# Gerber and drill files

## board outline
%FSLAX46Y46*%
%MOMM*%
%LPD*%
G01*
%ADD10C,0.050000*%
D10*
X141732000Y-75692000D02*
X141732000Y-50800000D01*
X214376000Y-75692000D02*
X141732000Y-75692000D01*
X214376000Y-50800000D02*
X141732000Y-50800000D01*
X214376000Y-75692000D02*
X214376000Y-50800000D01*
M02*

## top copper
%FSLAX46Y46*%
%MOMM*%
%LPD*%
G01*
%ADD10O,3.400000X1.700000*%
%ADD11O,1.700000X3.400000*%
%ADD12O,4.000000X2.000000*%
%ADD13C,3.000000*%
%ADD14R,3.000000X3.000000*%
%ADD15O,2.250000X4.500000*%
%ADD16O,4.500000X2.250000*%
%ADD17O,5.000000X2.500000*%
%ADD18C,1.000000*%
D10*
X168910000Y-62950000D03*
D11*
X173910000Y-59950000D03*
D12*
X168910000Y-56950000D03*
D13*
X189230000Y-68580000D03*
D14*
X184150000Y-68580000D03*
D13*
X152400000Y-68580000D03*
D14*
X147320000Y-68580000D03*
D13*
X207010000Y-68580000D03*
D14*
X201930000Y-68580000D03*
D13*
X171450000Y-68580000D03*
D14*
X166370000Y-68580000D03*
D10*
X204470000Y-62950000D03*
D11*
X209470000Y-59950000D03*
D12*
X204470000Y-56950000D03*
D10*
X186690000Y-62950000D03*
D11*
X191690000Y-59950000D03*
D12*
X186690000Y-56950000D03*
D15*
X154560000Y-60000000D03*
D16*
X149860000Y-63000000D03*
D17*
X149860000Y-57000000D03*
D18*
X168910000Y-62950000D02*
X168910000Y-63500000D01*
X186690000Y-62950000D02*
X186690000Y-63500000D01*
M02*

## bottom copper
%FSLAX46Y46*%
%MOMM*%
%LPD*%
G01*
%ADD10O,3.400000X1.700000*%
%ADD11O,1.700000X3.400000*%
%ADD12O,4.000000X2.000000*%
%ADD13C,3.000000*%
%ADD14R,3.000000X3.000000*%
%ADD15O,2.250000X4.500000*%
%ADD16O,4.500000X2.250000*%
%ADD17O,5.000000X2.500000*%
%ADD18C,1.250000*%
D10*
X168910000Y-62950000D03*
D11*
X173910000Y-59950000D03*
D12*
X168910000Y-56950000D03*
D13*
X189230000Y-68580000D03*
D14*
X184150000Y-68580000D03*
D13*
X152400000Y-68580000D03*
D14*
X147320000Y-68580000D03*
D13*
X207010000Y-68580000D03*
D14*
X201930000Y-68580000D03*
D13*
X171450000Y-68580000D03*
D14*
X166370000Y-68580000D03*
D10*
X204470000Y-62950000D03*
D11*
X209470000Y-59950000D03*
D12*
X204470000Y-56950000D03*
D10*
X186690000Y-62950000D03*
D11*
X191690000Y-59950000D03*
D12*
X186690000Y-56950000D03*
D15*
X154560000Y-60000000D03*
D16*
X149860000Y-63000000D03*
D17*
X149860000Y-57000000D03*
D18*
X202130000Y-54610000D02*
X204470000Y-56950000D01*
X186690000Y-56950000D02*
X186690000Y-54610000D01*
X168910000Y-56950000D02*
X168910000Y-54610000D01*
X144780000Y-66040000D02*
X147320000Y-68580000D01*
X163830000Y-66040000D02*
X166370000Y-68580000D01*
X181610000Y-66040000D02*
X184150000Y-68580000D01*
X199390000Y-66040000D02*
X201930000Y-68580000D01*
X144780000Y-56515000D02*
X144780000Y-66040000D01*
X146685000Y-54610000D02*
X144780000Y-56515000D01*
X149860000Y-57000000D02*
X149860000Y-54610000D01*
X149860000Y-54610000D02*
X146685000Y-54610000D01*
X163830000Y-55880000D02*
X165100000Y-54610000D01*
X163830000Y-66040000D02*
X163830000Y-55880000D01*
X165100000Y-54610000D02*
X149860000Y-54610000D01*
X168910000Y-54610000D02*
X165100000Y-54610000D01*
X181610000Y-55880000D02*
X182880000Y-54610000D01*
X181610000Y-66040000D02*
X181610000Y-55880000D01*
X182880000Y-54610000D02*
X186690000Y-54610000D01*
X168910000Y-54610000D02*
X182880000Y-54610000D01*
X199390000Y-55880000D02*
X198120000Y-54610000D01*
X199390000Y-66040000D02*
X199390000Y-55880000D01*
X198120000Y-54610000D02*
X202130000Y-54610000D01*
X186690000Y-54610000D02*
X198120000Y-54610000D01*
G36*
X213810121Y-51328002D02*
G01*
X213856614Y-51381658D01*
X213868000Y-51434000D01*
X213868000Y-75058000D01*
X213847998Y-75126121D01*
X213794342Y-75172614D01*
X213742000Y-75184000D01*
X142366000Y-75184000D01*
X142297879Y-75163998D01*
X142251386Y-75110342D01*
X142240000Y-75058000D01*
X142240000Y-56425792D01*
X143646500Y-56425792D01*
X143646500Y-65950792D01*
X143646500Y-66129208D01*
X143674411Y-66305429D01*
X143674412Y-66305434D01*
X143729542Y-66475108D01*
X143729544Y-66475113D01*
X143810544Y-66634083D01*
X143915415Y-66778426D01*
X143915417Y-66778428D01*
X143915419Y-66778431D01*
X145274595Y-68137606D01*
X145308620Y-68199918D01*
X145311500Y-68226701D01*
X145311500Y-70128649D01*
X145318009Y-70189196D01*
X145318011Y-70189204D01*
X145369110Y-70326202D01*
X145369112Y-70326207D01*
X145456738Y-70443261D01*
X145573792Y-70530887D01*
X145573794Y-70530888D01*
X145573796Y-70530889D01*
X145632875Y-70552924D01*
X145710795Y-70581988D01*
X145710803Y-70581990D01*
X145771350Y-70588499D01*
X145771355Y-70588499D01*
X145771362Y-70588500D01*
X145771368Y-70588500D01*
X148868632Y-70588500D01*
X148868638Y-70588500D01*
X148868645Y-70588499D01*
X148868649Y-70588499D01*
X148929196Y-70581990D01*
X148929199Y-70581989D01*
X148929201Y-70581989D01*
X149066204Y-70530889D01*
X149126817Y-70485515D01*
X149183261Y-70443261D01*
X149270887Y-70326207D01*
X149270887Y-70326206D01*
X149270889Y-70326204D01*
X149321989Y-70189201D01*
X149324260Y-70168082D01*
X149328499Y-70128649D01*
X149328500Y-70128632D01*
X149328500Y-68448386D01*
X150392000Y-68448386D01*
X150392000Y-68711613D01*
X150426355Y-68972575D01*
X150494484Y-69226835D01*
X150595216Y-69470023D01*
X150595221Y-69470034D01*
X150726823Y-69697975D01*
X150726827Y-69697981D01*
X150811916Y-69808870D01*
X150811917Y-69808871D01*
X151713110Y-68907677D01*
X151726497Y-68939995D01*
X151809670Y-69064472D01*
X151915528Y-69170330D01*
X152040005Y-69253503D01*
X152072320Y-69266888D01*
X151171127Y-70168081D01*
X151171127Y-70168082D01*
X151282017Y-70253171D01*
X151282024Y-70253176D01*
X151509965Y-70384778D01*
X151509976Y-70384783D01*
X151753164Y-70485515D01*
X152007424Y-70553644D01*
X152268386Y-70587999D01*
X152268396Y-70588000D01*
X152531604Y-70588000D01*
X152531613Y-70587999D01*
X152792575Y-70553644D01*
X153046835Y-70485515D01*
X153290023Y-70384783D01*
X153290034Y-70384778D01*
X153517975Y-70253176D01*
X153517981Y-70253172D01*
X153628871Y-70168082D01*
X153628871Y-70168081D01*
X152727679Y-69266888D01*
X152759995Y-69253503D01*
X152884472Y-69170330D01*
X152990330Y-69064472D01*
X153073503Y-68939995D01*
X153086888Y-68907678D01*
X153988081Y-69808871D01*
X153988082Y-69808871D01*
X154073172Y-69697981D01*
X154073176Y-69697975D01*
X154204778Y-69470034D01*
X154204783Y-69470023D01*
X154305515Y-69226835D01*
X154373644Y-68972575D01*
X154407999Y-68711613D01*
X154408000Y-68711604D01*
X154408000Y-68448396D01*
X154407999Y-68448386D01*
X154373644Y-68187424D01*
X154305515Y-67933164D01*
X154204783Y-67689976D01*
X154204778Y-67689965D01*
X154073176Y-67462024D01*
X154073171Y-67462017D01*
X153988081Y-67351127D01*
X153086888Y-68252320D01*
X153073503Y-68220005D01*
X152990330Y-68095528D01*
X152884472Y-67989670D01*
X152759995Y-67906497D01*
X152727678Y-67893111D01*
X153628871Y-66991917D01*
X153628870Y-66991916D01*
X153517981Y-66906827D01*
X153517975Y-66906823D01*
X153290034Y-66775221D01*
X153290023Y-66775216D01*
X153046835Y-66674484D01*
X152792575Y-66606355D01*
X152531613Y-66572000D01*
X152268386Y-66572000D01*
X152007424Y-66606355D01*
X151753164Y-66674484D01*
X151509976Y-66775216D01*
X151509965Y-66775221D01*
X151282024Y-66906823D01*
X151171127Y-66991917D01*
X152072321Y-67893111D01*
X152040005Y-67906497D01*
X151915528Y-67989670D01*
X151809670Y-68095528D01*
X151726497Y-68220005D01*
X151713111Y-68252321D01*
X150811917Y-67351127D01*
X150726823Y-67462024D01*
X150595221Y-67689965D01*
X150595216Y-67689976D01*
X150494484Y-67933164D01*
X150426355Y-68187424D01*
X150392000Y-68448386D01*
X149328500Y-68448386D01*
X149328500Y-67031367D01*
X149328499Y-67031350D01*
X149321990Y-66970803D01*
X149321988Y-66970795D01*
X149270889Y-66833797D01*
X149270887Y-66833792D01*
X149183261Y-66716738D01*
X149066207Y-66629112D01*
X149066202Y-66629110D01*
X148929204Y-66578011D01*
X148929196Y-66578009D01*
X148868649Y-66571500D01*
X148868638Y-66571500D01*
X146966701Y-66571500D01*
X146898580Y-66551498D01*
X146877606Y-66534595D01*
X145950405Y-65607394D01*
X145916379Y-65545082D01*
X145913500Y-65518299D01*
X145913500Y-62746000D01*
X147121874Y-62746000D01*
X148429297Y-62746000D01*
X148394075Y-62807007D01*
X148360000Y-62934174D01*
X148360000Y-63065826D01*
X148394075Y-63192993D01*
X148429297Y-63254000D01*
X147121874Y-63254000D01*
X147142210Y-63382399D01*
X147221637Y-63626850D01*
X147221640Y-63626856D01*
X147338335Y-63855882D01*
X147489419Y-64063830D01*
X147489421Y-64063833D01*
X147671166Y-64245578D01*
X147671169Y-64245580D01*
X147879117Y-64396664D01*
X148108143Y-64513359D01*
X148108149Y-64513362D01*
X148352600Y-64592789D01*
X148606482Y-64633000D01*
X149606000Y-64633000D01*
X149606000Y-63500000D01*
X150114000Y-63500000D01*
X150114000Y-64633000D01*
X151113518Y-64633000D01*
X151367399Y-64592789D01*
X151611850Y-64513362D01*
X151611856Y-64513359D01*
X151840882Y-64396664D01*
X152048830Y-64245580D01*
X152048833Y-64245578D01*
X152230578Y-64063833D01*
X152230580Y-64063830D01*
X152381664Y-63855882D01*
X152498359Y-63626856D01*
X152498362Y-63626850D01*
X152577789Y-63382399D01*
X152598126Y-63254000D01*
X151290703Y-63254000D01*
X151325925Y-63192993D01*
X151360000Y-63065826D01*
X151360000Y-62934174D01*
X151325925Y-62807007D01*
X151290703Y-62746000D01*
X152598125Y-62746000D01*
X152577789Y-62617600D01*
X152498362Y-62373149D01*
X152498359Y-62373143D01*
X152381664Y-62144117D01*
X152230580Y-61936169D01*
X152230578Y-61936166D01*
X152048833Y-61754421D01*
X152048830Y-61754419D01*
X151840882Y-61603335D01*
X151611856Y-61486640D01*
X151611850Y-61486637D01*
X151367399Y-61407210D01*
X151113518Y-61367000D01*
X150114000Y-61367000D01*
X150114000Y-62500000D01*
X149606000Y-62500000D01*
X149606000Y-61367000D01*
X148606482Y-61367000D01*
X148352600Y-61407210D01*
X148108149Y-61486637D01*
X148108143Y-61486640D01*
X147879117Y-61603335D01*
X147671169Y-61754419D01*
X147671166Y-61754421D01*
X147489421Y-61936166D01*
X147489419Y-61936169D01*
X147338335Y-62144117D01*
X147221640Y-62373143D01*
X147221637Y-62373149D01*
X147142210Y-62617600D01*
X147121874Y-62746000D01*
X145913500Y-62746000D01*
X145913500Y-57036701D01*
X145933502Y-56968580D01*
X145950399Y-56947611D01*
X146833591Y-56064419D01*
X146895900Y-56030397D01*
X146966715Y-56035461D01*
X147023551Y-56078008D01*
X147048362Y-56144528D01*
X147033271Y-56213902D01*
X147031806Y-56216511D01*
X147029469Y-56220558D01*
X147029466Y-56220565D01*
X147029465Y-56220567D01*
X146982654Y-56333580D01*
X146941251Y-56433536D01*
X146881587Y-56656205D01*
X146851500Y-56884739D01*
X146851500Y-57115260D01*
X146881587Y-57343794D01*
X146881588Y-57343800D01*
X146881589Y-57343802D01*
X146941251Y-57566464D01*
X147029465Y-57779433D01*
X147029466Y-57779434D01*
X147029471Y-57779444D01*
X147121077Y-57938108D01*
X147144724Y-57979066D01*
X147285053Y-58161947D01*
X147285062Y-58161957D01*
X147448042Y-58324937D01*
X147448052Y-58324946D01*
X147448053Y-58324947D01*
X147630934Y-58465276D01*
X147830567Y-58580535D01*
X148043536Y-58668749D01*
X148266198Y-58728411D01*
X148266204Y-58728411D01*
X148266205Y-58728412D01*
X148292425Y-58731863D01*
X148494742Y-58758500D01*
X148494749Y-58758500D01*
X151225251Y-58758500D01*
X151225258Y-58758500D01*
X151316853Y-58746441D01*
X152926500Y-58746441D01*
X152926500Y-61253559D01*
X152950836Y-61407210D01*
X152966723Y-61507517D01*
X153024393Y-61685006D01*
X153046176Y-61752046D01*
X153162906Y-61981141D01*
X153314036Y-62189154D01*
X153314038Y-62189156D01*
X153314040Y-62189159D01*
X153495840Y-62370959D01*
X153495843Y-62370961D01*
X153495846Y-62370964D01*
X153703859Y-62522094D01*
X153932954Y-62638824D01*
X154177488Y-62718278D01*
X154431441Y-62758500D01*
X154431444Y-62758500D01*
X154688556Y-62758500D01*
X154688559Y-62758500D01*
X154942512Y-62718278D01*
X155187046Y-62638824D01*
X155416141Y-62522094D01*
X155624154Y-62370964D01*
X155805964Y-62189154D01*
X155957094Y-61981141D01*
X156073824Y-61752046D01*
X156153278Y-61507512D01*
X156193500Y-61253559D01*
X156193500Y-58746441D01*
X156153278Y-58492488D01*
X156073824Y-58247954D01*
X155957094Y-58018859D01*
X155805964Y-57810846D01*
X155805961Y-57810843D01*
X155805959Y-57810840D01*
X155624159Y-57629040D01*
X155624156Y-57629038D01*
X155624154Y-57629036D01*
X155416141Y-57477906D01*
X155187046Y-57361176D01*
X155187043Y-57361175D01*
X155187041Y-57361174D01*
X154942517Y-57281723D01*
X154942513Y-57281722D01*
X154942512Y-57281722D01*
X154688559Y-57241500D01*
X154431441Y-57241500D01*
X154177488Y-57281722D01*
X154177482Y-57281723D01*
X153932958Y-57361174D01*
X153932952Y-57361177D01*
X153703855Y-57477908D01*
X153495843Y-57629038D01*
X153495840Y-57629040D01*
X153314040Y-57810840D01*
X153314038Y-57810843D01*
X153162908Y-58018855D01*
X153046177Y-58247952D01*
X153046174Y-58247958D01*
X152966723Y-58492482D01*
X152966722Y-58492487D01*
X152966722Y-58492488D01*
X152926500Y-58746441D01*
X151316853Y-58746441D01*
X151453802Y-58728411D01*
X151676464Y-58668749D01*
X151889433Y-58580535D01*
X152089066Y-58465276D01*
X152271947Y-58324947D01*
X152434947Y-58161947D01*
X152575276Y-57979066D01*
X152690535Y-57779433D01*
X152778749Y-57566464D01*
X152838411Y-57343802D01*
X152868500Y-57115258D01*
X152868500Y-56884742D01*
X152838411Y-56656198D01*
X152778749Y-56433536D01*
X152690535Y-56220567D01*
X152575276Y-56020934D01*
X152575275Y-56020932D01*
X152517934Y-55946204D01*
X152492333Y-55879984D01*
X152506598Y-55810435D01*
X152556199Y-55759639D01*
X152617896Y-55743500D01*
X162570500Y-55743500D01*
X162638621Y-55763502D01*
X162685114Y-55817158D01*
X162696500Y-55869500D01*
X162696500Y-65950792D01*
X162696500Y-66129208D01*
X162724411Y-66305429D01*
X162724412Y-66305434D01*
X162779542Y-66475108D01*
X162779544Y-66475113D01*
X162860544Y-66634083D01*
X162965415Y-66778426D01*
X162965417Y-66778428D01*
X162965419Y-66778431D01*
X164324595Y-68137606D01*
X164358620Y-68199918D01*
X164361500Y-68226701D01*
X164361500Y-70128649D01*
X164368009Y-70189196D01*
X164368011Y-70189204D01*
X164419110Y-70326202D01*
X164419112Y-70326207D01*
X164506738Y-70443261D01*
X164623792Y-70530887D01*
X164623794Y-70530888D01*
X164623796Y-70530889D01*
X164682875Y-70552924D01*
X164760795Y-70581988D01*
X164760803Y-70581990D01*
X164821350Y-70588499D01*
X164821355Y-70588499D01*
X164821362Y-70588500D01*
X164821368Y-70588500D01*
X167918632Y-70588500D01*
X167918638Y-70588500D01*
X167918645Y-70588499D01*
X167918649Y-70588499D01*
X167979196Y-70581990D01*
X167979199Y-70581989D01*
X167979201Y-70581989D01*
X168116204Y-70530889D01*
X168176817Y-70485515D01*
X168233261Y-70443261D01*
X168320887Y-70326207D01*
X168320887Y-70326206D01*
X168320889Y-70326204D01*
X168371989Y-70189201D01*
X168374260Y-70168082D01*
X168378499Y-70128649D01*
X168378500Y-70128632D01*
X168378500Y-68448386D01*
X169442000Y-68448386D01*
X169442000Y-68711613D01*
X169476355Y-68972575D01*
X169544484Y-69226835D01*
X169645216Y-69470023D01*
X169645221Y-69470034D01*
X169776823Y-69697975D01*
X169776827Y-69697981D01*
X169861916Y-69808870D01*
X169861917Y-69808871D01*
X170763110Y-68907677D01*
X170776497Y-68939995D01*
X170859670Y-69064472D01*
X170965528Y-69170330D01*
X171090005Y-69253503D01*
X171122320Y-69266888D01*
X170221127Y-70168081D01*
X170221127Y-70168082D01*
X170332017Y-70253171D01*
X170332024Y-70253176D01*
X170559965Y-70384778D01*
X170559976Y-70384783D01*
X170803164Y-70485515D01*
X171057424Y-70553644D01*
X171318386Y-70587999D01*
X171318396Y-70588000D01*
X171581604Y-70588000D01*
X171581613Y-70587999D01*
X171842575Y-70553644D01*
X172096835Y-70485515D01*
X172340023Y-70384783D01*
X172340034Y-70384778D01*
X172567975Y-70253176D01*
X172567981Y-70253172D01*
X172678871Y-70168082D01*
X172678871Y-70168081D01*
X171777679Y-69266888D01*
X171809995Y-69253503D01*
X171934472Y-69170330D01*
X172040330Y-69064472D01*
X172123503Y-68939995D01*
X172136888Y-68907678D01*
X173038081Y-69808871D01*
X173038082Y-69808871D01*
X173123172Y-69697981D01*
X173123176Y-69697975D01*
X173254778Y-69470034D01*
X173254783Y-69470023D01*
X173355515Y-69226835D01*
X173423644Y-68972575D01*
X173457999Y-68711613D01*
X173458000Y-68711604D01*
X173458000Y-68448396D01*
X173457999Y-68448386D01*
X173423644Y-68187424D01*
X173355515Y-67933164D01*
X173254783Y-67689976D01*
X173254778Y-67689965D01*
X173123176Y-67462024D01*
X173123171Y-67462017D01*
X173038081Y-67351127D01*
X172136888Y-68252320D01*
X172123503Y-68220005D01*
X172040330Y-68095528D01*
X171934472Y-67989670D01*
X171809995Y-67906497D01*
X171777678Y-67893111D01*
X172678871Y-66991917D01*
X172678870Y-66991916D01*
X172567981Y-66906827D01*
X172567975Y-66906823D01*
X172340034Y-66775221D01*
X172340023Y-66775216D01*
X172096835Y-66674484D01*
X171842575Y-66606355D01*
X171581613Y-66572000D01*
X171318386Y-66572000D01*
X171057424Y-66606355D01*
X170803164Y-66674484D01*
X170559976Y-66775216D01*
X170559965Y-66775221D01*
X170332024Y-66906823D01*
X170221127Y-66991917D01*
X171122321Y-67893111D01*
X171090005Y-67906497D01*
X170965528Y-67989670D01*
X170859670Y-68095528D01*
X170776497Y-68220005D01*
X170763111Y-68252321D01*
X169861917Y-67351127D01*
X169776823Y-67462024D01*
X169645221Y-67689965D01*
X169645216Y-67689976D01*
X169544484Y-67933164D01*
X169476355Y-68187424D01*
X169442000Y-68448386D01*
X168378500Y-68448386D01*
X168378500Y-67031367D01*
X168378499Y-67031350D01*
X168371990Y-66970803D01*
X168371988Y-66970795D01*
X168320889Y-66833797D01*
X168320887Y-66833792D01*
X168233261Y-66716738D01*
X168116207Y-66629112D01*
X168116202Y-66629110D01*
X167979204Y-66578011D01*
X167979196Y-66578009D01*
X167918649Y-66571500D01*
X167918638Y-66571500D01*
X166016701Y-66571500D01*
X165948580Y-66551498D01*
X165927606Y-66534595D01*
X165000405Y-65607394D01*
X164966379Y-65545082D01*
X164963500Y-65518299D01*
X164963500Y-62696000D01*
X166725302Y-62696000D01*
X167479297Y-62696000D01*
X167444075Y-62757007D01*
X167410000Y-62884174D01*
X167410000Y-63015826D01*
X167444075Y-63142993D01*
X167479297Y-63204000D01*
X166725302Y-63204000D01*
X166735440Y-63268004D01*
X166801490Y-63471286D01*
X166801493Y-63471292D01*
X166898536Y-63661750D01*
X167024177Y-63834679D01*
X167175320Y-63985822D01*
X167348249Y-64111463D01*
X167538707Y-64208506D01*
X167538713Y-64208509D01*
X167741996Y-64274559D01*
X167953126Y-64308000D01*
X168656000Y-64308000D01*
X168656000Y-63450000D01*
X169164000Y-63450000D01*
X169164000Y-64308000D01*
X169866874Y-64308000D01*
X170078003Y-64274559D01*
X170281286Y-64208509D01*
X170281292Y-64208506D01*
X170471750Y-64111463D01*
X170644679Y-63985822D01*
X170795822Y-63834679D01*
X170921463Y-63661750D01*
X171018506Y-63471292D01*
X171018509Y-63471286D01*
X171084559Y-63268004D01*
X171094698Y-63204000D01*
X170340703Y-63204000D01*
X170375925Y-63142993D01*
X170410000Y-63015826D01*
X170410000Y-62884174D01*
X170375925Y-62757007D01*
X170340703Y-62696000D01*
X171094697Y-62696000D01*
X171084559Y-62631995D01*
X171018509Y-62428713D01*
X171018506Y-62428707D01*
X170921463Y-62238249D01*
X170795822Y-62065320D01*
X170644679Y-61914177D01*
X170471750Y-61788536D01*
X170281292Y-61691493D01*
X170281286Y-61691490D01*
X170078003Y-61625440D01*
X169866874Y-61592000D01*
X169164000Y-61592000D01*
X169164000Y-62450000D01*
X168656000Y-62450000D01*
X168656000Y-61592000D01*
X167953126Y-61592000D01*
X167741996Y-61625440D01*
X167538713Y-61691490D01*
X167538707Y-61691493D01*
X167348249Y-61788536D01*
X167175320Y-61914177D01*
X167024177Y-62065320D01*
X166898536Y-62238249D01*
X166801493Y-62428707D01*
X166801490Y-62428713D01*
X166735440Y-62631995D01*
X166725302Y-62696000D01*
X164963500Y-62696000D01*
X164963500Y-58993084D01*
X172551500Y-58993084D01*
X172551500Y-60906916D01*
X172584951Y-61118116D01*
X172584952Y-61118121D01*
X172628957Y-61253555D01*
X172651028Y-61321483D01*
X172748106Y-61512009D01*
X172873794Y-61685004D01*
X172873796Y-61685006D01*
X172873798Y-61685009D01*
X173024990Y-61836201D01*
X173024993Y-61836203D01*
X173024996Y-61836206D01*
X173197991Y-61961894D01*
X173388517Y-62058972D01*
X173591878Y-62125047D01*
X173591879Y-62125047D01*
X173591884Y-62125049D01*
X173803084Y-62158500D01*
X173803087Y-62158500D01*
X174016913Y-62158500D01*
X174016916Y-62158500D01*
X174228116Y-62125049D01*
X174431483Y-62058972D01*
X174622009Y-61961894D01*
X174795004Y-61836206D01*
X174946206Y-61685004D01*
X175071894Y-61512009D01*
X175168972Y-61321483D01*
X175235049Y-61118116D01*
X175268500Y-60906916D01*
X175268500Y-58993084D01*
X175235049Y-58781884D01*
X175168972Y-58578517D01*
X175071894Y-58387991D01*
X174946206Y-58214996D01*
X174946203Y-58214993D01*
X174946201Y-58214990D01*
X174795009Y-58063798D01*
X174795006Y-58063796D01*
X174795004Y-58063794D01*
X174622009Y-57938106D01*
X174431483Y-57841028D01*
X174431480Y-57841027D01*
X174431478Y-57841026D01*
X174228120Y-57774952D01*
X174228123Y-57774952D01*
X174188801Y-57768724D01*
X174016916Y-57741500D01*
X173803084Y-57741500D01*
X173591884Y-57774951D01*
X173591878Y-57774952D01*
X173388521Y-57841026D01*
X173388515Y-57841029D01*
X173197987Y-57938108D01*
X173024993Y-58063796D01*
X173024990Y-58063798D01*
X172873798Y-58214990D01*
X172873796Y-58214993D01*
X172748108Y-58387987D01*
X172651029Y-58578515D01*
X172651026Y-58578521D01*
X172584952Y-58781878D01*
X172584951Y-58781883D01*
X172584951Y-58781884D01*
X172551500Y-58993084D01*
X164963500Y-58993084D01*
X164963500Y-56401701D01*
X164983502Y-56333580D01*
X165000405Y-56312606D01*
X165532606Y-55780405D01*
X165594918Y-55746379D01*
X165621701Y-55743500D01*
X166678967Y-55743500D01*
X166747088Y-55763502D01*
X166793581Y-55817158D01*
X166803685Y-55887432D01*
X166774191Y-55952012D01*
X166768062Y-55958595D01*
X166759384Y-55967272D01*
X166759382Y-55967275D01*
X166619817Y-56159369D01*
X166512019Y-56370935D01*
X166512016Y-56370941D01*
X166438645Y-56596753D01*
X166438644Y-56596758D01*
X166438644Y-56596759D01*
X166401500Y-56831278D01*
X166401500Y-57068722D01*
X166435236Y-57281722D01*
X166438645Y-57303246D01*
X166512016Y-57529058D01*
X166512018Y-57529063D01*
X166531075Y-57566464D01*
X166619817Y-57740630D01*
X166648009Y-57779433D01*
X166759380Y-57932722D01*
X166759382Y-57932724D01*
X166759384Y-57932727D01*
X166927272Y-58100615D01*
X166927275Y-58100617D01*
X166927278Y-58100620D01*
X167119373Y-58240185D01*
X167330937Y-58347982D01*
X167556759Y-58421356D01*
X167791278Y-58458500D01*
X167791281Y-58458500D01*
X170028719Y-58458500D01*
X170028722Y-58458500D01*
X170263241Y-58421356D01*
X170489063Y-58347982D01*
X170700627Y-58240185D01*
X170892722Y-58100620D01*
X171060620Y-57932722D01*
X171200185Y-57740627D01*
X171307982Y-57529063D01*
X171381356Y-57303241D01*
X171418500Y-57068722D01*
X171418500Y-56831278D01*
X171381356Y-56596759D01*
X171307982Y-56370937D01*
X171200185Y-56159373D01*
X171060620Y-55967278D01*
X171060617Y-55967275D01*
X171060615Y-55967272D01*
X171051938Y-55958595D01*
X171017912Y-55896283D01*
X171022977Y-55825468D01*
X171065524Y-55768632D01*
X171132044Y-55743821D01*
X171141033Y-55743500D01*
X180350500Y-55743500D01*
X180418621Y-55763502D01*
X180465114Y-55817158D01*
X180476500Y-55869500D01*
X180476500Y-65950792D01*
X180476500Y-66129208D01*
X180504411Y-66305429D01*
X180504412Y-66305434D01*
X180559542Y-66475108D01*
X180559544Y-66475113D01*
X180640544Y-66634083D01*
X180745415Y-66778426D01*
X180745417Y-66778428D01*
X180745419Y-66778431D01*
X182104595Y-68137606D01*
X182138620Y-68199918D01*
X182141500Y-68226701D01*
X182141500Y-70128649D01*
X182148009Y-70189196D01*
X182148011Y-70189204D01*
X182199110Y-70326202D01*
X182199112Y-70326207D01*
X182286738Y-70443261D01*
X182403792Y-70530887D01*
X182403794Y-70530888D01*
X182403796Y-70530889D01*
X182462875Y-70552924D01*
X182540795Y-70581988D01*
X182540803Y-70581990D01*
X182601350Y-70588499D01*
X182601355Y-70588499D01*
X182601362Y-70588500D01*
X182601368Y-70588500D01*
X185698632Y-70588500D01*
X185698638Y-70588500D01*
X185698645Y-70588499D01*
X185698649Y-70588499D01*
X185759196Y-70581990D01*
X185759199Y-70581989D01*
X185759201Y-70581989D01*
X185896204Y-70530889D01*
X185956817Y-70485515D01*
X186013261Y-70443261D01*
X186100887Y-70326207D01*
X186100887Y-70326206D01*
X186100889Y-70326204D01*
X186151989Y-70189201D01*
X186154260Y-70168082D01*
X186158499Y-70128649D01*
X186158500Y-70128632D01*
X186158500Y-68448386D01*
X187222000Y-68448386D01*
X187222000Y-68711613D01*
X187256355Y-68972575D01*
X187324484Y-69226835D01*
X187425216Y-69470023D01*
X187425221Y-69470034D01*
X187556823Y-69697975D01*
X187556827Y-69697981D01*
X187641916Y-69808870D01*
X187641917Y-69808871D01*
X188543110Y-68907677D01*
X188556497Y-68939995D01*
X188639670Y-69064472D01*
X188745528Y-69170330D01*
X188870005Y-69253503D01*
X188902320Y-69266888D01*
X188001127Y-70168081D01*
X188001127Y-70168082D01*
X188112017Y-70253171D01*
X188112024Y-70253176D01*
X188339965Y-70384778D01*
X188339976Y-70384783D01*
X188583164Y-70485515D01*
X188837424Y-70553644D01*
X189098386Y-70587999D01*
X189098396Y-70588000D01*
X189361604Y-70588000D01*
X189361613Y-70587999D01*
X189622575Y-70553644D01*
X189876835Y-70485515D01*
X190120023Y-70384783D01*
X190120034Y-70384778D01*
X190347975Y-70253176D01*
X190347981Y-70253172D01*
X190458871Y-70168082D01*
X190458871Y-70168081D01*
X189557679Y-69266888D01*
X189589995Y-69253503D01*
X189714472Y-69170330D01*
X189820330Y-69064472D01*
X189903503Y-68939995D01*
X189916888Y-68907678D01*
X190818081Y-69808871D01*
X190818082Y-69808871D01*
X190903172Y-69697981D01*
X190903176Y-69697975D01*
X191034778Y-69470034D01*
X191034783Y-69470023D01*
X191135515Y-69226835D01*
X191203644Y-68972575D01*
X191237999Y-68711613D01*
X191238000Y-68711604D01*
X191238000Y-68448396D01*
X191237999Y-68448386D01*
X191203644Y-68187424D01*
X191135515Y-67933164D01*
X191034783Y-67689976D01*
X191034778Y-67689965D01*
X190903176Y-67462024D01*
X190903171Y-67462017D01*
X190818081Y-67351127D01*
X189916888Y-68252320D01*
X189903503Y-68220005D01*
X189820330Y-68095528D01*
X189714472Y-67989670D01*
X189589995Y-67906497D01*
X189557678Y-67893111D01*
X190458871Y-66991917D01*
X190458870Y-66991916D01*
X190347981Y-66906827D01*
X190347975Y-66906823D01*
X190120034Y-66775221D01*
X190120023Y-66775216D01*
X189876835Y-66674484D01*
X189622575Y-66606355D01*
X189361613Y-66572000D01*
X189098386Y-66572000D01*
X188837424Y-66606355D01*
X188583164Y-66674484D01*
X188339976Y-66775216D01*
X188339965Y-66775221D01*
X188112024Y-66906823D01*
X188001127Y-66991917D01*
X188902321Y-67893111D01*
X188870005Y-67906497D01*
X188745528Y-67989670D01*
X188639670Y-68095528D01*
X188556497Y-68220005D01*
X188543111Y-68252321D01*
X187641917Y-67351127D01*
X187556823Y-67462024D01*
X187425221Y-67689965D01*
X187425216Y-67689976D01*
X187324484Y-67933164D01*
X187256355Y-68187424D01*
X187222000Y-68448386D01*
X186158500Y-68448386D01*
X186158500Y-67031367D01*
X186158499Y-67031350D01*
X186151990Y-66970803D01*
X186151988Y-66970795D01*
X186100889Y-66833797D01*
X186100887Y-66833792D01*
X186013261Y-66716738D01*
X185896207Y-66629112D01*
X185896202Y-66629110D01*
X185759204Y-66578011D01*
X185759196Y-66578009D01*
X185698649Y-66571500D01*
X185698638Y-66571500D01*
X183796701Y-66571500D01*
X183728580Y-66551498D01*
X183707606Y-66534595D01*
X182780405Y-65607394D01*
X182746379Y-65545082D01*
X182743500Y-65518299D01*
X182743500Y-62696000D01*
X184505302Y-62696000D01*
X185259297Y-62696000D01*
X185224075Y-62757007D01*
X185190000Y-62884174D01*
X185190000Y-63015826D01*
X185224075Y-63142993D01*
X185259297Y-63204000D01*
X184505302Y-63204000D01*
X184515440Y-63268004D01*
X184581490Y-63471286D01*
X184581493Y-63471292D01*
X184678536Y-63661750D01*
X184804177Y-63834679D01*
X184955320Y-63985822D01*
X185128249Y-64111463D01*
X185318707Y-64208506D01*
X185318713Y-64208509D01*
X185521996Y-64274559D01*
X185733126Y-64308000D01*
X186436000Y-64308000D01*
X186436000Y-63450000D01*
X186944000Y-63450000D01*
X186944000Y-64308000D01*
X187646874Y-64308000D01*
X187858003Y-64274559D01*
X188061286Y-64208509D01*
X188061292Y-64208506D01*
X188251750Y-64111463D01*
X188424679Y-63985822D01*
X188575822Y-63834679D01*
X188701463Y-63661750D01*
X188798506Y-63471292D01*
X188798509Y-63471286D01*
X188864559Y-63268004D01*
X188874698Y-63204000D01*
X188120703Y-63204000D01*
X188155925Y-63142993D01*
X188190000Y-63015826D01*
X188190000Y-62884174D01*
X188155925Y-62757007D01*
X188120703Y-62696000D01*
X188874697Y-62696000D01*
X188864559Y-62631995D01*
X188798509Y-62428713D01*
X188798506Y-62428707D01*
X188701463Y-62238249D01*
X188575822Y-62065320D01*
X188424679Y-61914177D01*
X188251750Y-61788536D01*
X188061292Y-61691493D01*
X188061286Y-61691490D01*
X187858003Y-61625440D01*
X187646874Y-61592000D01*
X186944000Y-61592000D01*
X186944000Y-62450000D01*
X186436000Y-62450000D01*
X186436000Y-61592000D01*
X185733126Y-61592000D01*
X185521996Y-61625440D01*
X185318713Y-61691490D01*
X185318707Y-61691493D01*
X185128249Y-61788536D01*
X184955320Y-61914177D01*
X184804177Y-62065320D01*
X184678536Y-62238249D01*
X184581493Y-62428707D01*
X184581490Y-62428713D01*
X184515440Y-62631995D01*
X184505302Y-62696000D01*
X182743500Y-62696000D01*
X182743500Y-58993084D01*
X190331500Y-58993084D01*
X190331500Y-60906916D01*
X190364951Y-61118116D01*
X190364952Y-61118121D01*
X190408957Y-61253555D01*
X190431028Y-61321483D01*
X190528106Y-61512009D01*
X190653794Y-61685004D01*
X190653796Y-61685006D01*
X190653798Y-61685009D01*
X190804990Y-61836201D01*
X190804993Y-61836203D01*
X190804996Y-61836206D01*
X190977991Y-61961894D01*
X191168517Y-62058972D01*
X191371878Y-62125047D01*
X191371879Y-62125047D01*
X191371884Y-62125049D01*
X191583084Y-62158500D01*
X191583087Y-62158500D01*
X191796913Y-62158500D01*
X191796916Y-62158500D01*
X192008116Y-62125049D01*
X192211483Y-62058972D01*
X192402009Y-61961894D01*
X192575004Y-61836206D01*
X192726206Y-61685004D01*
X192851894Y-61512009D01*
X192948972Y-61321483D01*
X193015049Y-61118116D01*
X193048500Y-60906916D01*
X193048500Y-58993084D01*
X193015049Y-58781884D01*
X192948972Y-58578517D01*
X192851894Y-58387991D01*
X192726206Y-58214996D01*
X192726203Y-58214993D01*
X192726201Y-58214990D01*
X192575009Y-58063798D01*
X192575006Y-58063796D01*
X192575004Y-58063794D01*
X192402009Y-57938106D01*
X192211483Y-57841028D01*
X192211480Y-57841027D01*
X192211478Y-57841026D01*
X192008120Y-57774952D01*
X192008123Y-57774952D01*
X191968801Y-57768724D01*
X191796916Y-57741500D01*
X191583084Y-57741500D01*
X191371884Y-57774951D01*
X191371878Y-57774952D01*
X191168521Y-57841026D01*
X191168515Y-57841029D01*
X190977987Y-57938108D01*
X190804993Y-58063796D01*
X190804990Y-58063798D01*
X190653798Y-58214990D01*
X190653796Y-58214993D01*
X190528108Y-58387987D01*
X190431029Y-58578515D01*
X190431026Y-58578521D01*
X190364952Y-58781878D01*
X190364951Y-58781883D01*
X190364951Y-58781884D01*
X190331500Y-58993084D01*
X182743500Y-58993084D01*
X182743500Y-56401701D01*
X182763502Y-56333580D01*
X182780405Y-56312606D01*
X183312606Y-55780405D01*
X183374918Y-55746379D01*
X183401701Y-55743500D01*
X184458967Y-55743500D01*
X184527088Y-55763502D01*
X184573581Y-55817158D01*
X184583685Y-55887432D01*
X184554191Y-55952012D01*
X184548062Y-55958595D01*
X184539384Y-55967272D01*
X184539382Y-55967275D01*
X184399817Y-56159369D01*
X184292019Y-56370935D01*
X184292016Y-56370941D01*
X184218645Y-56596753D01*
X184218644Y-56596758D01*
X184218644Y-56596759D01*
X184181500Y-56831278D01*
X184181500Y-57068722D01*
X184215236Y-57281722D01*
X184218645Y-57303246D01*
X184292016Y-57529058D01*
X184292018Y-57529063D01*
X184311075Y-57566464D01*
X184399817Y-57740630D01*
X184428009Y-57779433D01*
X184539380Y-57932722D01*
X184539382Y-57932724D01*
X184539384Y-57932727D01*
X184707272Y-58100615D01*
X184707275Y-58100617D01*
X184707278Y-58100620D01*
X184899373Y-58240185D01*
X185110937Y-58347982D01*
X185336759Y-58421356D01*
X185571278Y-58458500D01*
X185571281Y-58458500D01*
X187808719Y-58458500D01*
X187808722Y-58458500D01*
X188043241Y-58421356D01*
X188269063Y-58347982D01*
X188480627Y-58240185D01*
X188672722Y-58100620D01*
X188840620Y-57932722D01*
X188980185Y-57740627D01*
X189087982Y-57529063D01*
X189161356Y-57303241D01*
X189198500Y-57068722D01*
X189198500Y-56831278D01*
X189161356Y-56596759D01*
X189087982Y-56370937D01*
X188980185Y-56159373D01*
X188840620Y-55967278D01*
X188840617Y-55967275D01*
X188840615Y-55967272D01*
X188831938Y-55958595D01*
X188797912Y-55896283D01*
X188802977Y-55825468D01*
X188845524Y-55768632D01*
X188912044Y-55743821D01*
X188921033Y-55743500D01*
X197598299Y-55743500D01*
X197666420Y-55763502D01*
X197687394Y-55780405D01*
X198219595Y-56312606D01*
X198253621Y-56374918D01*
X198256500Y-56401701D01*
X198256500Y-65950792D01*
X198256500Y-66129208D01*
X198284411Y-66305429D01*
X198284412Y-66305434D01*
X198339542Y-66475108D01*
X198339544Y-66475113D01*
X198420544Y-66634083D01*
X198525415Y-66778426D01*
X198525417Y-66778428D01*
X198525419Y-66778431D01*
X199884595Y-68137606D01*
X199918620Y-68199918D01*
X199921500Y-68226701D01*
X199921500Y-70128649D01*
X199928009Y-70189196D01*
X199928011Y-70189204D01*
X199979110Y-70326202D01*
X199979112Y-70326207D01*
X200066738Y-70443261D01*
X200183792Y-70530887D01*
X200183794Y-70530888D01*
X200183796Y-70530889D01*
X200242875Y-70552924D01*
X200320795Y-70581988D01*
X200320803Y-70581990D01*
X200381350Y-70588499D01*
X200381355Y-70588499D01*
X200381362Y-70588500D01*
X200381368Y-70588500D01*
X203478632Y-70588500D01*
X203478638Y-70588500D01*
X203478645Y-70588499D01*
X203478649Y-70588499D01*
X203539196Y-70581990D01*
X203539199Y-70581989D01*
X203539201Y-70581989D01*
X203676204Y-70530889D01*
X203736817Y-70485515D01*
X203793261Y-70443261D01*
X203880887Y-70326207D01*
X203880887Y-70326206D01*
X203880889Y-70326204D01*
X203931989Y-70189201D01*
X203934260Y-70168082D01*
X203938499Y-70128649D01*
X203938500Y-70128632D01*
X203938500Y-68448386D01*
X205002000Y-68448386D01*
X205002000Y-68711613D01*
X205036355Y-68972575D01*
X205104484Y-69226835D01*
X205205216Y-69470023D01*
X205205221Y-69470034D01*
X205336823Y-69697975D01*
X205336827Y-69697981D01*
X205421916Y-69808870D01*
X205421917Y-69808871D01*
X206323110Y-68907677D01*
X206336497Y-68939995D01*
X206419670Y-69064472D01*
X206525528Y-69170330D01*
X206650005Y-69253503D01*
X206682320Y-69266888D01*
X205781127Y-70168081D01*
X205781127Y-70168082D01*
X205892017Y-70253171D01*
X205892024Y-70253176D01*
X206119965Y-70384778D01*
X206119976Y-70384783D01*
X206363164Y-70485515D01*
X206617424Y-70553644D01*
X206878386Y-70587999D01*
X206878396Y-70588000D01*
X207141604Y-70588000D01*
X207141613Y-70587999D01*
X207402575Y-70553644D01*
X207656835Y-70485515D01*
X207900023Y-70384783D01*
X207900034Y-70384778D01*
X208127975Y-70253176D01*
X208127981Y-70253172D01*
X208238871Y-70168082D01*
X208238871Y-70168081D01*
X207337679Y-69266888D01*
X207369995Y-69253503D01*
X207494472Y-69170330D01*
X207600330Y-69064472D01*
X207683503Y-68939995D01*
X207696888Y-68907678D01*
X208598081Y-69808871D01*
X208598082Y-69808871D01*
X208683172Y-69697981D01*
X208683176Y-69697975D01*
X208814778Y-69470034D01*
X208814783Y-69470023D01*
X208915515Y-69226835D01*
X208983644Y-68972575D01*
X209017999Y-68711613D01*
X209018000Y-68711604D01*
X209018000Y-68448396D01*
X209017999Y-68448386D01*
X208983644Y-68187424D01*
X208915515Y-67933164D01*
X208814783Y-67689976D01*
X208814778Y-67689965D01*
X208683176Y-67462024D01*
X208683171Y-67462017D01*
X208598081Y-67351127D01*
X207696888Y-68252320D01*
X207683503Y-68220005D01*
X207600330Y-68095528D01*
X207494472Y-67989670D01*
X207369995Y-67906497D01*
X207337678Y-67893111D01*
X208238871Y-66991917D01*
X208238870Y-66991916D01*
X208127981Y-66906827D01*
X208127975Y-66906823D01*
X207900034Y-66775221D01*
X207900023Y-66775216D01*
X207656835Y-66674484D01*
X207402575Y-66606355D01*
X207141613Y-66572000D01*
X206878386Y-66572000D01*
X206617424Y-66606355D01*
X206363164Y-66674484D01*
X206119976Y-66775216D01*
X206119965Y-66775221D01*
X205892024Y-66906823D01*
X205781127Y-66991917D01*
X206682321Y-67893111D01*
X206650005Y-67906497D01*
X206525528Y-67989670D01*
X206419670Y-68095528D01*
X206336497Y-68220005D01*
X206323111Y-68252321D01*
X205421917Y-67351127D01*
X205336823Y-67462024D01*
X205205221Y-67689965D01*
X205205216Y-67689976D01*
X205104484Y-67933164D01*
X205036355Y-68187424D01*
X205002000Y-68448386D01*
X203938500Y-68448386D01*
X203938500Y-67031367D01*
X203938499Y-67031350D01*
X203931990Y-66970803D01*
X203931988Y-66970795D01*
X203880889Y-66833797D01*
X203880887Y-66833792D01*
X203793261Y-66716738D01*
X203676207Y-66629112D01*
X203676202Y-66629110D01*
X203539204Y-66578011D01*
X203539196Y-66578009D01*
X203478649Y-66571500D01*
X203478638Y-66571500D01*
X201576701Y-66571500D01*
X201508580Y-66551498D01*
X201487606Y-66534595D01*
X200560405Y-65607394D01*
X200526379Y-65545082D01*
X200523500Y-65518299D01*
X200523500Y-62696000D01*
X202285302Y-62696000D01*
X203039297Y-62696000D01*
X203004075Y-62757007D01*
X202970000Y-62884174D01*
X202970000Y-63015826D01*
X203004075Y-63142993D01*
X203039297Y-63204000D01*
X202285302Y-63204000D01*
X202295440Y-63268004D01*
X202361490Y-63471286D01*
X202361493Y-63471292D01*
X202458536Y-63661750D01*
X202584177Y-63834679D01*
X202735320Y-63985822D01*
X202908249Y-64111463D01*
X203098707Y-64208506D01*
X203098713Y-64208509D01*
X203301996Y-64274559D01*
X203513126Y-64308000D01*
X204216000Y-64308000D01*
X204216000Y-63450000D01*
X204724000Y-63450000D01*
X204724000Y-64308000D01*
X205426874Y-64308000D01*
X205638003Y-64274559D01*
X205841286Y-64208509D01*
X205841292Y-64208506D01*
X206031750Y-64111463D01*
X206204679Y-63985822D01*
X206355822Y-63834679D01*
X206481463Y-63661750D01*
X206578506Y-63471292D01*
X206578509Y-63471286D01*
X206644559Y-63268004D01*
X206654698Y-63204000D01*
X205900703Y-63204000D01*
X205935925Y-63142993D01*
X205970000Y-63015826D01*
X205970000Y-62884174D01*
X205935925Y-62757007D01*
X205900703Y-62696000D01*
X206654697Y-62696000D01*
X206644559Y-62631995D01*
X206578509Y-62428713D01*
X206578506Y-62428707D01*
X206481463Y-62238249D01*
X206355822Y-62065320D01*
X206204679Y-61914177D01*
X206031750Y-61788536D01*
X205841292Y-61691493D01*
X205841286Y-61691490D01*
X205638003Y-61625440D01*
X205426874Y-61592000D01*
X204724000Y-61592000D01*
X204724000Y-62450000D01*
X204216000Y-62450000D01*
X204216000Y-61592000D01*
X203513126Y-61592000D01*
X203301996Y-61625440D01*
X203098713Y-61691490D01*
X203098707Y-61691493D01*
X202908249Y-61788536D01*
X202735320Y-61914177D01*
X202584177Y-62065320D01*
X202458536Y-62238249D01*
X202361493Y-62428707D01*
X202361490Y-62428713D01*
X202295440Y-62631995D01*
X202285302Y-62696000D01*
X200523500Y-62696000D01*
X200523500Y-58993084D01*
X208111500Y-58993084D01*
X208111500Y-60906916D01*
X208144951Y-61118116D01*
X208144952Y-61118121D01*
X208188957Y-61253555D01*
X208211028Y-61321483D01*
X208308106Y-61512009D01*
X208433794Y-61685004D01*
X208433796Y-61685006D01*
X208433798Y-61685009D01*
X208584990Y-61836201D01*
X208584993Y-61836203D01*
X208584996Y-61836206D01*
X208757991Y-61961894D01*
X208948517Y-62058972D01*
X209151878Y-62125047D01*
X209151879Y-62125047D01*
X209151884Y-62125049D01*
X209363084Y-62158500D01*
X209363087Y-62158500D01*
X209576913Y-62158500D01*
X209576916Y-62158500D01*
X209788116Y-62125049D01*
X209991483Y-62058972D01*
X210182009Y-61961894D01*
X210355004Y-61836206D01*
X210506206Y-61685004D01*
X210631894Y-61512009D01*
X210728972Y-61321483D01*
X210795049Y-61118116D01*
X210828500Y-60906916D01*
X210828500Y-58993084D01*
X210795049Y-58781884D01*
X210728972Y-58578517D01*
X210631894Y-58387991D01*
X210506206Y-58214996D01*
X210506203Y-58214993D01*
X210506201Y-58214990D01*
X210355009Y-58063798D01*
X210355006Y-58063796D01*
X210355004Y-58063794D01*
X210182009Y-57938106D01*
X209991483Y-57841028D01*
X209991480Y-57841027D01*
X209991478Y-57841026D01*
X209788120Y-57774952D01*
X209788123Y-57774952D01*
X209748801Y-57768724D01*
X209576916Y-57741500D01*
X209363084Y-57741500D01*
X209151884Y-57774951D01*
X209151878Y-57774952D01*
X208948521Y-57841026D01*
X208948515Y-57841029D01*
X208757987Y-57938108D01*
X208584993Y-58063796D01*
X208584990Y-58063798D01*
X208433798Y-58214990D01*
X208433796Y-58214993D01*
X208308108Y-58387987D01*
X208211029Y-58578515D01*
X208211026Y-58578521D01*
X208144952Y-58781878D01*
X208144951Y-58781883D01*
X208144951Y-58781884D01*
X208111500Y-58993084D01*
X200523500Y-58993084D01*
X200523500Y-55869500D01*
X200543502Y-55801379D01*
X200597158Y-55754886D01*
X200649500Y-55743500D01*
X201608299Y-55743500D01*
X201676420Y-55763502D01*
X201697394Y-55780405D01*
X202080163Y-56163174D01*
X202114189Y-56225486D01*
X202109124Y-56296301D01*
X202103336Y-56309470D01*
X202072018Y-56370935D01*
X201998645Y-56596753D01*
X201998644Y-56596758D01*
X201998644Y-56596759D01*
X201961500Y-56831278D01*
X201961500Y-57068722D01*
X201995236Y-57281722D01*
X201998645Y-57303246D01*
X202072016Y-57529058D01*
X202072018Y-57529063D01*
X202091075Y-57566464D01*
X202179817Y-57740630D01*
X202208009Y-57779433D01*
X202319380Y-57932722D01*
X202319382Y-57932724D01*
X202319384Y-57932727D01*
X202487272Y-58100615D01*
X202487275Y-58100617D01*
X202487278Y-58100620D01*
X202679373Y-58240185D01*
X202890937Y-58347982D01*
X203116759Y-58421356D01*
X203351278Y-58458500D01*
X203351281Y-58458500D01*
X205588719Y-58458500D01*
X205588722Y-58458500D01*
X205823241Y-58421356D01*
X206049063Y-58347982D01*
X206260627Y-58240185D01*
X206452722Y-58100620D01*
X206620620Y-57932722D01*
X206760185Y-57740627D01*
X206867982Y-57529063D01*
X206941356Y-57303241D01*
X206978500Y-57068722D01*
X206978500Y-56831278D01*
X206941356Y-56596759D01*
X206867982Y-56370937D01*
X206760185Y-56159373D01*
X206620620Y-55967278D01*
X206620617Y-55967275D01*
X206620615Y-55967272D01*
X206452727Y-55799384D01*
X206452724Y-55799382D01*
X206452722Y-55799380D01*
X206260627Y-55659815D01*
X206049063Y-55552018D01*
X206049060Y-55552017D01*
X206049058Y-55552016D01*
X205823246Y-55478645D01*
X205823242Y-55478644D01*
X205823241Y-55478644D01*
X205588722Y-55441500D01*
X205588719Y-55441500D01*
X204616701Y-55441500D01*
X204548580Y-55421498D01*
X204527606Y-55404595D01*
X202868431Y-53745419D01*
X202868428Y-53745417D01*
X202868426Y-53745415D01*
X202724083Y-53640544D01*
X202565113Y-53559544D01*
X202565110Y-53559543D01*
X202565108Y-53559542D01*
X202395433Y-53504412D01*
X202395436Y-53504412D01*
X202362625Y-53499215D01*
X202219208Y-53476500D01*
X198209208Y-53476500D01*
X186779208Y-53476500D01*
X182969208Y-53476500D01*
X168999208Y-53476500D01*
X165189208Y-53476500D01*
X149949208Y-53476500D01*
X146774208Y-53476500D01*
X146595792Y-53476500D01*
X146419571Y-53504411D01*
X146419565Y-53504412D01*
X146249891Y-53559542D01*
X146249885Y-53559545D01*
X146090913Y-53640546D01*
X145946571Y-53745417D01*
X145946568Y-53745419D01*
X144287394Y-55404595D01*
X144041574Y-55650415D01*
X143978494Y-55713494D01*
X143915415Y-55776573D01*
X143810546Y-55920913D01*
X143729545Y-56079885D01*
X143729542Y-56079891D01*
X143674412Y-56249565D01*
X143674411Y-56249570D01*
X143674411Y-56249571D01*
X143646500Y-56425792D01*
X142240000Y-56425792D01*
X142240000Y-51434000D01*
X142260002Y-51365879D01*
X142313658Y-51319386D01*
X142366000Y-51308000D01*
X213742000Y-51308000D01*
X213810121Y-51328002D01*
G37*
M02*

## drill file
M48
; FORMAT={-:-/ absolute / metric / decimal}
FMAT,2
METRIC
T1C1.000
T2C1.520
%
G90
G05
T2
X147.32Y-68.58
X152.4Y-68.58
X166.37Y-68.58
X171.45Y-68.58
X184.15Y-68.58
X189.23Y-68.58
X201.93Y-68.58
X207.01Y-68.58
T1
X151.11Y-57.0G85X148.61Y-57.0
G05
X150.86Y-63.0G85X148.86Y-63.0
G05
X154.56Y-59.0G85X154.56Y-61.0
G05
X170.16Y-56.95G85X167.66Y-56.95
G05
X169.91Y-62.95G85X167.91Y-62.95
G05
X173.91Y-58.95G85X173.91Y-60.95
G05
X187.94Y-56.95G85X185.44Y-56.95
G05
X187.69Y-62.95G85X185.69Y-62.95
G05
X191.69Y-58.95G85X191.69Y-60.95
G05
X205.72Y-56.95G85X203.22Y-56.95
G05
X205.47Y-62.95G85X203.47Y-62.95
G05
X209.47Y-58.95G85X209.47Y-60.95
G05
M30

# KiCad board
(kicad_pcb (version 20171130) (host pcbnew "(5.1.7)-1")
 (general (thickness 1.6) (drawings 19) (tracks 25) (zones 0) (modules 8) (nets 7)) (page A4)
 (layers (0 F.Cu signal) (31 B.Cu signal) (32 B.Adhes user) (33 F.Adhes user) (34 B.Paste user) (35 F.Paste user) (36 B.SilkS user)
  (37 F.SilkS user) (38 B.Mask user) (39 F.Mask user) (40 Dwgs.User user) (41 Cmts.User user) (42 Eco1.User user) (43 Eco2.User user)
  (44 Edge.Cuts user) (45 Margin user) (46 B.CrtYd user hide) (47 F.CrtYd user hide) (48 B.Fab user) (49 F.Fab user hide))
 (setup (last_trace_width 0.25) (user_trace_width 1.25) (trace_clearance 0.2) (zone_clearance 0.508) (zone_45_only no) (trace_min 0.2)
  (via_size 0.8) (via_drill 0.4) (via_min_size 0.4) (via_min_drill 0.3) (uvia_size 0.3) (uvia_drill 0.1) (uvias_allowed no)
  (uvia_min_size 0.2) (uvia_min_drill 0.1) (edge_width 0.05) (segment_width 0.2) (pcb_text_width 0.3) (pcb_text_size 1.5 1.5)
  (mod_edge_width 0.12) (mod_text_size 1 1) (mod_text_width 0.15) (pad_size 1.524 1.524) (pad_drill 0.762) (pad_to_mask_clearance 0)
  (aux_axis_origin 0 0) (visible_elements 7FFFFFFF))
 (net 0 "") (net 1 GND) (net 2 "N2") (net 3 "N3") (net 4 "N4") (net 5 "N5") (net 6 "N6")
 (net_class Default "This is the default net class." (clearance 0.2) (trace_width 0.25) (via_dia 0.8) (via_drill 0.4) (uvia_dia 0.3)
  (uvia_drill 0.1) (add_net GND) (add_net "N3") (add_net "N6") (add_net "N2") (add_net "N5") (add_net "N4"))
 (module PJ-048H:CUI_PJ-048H (layer F.Cu) (at 168.91 63.5 270)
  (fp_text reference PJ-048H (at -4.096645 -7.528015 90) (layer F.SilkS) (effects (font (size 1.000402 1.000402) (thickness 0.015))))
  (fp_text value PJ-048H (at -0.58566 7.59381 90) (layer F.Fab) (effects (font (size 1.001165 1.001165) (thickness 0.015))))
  (pad 2 thru_hole oval (at -0.55 0 270) (size 1.7 3.4) (drill oval 1 3) (layers *.Cu *.Mask) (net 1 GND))
  (pad 3 thru_hole oval (at -3.55 -5 270) (size 3.4 1.7) (drill oval 3 1) (layers *.Cu *.Mask) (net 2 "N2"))
  (pad 1 thru_hole oval (at -6.55 0 270) (size 2 4) (drill oval 1 3.5) (layers *.Cu *.Mask) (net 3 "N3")))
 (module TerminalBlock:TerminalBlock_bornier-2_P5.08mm (layer F.Cu) (at 184.15 68.58)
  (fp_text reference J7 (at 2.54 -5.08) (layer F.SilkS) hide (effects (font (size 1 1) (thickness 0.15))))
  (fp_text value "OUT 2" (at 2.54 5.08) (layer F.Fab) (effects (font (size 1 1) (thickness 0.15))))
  (pad 2 thru_hole circle (at 5.08 0) (size 3 3) (drill 1.52) (layers *.Cu *.Mask) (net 1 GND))
  (pad 1 thru_hole rect (at 0 0) (size 3 3) (drill 1.52) (layers *.Cu *.Mask) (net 3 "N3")))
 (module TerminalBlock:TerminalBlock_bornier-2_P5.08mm (layer F.Cu) (at 147.32 68.58)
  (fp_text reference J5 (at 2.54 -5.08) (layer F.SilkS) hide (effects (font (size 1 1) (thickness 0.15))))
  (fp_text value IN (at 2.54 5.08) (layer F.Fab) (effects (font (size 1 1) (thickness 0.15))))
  (pad 2 thru_hole circle (at 5.08 0) (size 3 3) (drill 1.52) (layers *.Cu *.Mask) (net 1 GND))
  (pad 1 thru_hole rect (at 0 0) (size 3 3) (drill 1.52) (layers *.Cu *.Mask) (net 3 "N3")))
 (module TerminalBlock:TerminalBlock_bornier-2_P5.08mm (layer F.Cu) (at 201.93 68.58)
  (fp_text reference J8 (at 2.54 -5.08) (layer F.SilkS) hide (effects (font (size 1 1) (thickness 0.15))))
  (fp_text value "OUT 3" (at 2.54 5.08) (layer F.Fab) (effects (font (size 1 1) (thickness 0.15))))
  (pad 2 thru_hole circle (at 5.08 0) (size 3 3) (drill 1.52) (layers *.Cu *.Mask) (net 1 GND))
  (pad 1 thru_hole rect (at 0 0) (size 3 3) (drill 1.52) (layers *.Cu *.Mask) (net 3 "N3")))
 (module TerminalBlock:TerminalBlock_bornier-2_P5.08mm (layer F.Cu) (at 166.37 68.58)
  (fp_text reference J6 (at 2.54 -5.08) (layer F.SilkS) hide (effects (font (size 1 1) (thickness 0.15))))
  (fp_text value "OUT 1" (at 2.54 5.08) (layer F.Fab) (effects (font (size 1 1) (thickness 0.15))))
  (pad 2 thru_hole circle (at 5.08 0) (size 3 3) (drill 1.52) (layers *.Cu *.Mask) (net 1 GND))
  (pad 1 thru_hole rect (at 0 0) (size 3 3) (drill 1.52) (layers *.Cu *.Mask) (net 3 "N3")))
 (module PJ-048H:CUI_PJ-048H (layer F.Cu) (at 204.47 63.5 270)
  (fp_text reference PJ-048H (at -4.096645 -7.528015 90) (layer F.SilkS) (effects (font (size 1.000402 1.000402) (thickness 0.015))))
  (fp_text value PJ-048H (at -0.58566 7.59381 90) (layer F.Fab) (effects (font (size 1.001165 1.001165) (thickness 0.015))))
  (pad 2 thru_hole oval (at -0.55 0 270) (size 1.7 3.4) (drill oval 1 3) (layers *.Cu *.Mask) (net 1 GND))
  (pad 3 thru_hole oval (at -3.55 -5 270) (size 3.4 1.7) (drill oval 3 1) (layers *.Cu *.Mask) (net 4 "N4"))
  (pad 1 thru_hole oval (at -6.55 0 270) (size 2 4) (drill oval 1 3.5) (layers *.Cu *.Mask) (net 3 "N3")))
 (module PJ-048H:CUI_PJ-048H (layer F.Cu) (at 186.69 63.5 270)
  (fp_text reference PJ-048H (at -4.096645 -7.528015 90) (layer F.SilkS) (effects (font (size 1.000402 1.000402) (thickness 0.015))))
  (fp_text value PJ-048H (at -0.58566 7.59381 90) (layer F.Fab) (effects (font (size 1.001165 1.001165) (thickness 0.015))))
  (pad 2 thru_hole oval (at -0.55 0 270) (size 1.7 3.4) (drill oval 1 3) (layers *.Cu *.Mask) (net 1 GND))
  (pad 3 thru_hole oval (at -3.55 -5 270) (size 3.4 1.7) (drill oval 3 1) (layers *.Cu *.Mask) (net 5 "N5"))
  (pad 1 thru_hole oval (at -6.55 0 270) (size 2 4) (drill oval 1 3.5) (layers *.Cu *.Mask) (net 3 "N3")))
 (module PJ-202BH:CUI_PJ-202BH (layer F.Cu) (at 149.86 63.5 270)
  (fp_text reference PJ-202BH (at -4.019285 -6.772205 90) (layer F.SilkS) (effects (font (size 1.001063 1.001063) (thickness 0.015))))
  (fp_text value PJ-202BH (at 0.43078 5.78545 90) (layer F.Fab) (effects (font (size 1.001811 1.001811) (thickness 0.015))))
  (pad 3 thru_hole oval (at -3.5 -4.7 270) (size 4.5 2.25) (drill oval 3 1) (layers *.Cu *.Mask) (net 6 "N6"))
  (pad 2 thru_hole oval (at -0.5 0 270) (size 2.25 4.5) (drill oval 1 3) (layers *.Cu *.Mask) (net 1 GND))
  (pad 1 thru_hole oval (at -6.5 0 270) (size 2.5 5) (drill oval 1 3.5) (layers *.Cu *.Mask) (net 3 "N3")))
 (gr_line (start 141.732 75.692) (end 141.732 50.8) (layer Edge.Cuts) (width 0.05))
 (gr_line (start 214.376 75.692) (end 141.732 75.692) (layer Edge.Cuts) (width 0.05))
 (gr_line (start 214.376 50.8) (end 141.732 50.8) (layer Edge.Cuts) (width 0.05))
 (gr_line (start 214.376 75.692) (end 214.376 50.8) (layer Edge.Cuts) (width 0.05))
 (segment (start 168.91 62.95) (end 168.91 63.5) (width 1) (layer F.Cu) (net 1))
 (segment (start 186.69 62.95) (end 186.69 63.5) (width 1) (layer F.Cu) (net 1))
 (segment (start 202.13 54.61) (end 204.47 56.95) (width 1.25) (layer B.Cu) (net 3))
 (segment (start 186.69 56.95) (end 186.69 54.61) (width 1.25) (layer B.Cu) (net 3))
 (segment (start 168.91 56.95) (end 168.91 54.61) (width 1.25) (layer B.Cu) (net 3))
 (segment (start 144.78 66.04) (end 147.32 68.58) (width 1.25) (layer B.Cu) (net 3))
 (segment (start 163.83 66.04) (end 166.37 68.58) (width 1.25) (layer B.Cu) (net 3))
 (segment (start 181.61 66.04) (end 184.15 68.58) (width 1.25) (layer B.Cu) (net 3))
 (segment (start 199.39 66.04) (end 201.93 68.58) (width 1.25) (layer B.Cu) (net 3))
 (segment (start 144.78 56.515) (end 144.78 66.04) (width 1.25) (layer B.Cu) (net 3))
 (segment (start 146.685 54.61) (end 144.78 56.515) (width 1.25) (layer B.Cu) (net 3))
 (segment (start 149.86 57) (end 149.86 54.61) (width 1.25) (layer B.Cu) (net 3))
 (segment (start 149.86 54.61) (end 146.685 54.61) (width 1.25) (layer B.Cu) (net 3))
 (segment (start 163.83 55.88) (end 165.1 54.61) (width 1.25) (layer B.Cu) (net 3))
 (segment (start 163.83 66.04) (end 163.83 55.88) (width 1.25) (layer B.Cu) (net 3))
 (segment (start 165.1 54.61) (end 149.86 54.61) (width 1.25) (layer B.Cu) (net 3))
 (segment (start 168.91 54.61) (end 165.1 54.61) (width 1.25) (layer B.Cu) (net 3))
 (segment (start 181.61 55.88) (end 182.88 54.61) (width 1.25) (layer B.Cu) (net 3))
 (segment (start 181.61 66.04) (end 181.61 55.88) (width 1.25) (layer B.Cu) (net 3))
 (segment (start 182.88 54.61) (end 186.69 54.61) (width 1.25) (layer B.Cu) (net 3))
 (segment (start 168.91 54.61) (end 182.88 54.61) (width 1.25) (layer B.Cu) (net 3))
 (segment (start 199.39 55.88) (end 198.12 54.61) (width 1.25) (layer B.Cu) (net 3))
 (segment (start 199.39 66.04) (end 199.39 55.88) (width 1.25) (layer B.Cu) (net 3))
 (segment (start 198.12 54.61) (end 202.13 54.61) (width 1.25) (layer B.Cu) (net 3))
 (segment (start 186.69 54.61) (end 198.12 54.61) (width 1.25) (layer B.Cu) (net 3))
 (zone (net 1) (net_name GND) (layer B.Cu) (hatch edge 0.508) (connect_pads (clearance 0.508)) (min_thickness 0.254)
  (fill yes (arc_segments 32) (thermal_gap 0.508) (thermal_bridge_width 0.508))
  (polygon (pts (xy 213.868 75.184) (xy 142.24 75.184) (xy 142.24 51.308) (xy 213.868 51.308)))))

